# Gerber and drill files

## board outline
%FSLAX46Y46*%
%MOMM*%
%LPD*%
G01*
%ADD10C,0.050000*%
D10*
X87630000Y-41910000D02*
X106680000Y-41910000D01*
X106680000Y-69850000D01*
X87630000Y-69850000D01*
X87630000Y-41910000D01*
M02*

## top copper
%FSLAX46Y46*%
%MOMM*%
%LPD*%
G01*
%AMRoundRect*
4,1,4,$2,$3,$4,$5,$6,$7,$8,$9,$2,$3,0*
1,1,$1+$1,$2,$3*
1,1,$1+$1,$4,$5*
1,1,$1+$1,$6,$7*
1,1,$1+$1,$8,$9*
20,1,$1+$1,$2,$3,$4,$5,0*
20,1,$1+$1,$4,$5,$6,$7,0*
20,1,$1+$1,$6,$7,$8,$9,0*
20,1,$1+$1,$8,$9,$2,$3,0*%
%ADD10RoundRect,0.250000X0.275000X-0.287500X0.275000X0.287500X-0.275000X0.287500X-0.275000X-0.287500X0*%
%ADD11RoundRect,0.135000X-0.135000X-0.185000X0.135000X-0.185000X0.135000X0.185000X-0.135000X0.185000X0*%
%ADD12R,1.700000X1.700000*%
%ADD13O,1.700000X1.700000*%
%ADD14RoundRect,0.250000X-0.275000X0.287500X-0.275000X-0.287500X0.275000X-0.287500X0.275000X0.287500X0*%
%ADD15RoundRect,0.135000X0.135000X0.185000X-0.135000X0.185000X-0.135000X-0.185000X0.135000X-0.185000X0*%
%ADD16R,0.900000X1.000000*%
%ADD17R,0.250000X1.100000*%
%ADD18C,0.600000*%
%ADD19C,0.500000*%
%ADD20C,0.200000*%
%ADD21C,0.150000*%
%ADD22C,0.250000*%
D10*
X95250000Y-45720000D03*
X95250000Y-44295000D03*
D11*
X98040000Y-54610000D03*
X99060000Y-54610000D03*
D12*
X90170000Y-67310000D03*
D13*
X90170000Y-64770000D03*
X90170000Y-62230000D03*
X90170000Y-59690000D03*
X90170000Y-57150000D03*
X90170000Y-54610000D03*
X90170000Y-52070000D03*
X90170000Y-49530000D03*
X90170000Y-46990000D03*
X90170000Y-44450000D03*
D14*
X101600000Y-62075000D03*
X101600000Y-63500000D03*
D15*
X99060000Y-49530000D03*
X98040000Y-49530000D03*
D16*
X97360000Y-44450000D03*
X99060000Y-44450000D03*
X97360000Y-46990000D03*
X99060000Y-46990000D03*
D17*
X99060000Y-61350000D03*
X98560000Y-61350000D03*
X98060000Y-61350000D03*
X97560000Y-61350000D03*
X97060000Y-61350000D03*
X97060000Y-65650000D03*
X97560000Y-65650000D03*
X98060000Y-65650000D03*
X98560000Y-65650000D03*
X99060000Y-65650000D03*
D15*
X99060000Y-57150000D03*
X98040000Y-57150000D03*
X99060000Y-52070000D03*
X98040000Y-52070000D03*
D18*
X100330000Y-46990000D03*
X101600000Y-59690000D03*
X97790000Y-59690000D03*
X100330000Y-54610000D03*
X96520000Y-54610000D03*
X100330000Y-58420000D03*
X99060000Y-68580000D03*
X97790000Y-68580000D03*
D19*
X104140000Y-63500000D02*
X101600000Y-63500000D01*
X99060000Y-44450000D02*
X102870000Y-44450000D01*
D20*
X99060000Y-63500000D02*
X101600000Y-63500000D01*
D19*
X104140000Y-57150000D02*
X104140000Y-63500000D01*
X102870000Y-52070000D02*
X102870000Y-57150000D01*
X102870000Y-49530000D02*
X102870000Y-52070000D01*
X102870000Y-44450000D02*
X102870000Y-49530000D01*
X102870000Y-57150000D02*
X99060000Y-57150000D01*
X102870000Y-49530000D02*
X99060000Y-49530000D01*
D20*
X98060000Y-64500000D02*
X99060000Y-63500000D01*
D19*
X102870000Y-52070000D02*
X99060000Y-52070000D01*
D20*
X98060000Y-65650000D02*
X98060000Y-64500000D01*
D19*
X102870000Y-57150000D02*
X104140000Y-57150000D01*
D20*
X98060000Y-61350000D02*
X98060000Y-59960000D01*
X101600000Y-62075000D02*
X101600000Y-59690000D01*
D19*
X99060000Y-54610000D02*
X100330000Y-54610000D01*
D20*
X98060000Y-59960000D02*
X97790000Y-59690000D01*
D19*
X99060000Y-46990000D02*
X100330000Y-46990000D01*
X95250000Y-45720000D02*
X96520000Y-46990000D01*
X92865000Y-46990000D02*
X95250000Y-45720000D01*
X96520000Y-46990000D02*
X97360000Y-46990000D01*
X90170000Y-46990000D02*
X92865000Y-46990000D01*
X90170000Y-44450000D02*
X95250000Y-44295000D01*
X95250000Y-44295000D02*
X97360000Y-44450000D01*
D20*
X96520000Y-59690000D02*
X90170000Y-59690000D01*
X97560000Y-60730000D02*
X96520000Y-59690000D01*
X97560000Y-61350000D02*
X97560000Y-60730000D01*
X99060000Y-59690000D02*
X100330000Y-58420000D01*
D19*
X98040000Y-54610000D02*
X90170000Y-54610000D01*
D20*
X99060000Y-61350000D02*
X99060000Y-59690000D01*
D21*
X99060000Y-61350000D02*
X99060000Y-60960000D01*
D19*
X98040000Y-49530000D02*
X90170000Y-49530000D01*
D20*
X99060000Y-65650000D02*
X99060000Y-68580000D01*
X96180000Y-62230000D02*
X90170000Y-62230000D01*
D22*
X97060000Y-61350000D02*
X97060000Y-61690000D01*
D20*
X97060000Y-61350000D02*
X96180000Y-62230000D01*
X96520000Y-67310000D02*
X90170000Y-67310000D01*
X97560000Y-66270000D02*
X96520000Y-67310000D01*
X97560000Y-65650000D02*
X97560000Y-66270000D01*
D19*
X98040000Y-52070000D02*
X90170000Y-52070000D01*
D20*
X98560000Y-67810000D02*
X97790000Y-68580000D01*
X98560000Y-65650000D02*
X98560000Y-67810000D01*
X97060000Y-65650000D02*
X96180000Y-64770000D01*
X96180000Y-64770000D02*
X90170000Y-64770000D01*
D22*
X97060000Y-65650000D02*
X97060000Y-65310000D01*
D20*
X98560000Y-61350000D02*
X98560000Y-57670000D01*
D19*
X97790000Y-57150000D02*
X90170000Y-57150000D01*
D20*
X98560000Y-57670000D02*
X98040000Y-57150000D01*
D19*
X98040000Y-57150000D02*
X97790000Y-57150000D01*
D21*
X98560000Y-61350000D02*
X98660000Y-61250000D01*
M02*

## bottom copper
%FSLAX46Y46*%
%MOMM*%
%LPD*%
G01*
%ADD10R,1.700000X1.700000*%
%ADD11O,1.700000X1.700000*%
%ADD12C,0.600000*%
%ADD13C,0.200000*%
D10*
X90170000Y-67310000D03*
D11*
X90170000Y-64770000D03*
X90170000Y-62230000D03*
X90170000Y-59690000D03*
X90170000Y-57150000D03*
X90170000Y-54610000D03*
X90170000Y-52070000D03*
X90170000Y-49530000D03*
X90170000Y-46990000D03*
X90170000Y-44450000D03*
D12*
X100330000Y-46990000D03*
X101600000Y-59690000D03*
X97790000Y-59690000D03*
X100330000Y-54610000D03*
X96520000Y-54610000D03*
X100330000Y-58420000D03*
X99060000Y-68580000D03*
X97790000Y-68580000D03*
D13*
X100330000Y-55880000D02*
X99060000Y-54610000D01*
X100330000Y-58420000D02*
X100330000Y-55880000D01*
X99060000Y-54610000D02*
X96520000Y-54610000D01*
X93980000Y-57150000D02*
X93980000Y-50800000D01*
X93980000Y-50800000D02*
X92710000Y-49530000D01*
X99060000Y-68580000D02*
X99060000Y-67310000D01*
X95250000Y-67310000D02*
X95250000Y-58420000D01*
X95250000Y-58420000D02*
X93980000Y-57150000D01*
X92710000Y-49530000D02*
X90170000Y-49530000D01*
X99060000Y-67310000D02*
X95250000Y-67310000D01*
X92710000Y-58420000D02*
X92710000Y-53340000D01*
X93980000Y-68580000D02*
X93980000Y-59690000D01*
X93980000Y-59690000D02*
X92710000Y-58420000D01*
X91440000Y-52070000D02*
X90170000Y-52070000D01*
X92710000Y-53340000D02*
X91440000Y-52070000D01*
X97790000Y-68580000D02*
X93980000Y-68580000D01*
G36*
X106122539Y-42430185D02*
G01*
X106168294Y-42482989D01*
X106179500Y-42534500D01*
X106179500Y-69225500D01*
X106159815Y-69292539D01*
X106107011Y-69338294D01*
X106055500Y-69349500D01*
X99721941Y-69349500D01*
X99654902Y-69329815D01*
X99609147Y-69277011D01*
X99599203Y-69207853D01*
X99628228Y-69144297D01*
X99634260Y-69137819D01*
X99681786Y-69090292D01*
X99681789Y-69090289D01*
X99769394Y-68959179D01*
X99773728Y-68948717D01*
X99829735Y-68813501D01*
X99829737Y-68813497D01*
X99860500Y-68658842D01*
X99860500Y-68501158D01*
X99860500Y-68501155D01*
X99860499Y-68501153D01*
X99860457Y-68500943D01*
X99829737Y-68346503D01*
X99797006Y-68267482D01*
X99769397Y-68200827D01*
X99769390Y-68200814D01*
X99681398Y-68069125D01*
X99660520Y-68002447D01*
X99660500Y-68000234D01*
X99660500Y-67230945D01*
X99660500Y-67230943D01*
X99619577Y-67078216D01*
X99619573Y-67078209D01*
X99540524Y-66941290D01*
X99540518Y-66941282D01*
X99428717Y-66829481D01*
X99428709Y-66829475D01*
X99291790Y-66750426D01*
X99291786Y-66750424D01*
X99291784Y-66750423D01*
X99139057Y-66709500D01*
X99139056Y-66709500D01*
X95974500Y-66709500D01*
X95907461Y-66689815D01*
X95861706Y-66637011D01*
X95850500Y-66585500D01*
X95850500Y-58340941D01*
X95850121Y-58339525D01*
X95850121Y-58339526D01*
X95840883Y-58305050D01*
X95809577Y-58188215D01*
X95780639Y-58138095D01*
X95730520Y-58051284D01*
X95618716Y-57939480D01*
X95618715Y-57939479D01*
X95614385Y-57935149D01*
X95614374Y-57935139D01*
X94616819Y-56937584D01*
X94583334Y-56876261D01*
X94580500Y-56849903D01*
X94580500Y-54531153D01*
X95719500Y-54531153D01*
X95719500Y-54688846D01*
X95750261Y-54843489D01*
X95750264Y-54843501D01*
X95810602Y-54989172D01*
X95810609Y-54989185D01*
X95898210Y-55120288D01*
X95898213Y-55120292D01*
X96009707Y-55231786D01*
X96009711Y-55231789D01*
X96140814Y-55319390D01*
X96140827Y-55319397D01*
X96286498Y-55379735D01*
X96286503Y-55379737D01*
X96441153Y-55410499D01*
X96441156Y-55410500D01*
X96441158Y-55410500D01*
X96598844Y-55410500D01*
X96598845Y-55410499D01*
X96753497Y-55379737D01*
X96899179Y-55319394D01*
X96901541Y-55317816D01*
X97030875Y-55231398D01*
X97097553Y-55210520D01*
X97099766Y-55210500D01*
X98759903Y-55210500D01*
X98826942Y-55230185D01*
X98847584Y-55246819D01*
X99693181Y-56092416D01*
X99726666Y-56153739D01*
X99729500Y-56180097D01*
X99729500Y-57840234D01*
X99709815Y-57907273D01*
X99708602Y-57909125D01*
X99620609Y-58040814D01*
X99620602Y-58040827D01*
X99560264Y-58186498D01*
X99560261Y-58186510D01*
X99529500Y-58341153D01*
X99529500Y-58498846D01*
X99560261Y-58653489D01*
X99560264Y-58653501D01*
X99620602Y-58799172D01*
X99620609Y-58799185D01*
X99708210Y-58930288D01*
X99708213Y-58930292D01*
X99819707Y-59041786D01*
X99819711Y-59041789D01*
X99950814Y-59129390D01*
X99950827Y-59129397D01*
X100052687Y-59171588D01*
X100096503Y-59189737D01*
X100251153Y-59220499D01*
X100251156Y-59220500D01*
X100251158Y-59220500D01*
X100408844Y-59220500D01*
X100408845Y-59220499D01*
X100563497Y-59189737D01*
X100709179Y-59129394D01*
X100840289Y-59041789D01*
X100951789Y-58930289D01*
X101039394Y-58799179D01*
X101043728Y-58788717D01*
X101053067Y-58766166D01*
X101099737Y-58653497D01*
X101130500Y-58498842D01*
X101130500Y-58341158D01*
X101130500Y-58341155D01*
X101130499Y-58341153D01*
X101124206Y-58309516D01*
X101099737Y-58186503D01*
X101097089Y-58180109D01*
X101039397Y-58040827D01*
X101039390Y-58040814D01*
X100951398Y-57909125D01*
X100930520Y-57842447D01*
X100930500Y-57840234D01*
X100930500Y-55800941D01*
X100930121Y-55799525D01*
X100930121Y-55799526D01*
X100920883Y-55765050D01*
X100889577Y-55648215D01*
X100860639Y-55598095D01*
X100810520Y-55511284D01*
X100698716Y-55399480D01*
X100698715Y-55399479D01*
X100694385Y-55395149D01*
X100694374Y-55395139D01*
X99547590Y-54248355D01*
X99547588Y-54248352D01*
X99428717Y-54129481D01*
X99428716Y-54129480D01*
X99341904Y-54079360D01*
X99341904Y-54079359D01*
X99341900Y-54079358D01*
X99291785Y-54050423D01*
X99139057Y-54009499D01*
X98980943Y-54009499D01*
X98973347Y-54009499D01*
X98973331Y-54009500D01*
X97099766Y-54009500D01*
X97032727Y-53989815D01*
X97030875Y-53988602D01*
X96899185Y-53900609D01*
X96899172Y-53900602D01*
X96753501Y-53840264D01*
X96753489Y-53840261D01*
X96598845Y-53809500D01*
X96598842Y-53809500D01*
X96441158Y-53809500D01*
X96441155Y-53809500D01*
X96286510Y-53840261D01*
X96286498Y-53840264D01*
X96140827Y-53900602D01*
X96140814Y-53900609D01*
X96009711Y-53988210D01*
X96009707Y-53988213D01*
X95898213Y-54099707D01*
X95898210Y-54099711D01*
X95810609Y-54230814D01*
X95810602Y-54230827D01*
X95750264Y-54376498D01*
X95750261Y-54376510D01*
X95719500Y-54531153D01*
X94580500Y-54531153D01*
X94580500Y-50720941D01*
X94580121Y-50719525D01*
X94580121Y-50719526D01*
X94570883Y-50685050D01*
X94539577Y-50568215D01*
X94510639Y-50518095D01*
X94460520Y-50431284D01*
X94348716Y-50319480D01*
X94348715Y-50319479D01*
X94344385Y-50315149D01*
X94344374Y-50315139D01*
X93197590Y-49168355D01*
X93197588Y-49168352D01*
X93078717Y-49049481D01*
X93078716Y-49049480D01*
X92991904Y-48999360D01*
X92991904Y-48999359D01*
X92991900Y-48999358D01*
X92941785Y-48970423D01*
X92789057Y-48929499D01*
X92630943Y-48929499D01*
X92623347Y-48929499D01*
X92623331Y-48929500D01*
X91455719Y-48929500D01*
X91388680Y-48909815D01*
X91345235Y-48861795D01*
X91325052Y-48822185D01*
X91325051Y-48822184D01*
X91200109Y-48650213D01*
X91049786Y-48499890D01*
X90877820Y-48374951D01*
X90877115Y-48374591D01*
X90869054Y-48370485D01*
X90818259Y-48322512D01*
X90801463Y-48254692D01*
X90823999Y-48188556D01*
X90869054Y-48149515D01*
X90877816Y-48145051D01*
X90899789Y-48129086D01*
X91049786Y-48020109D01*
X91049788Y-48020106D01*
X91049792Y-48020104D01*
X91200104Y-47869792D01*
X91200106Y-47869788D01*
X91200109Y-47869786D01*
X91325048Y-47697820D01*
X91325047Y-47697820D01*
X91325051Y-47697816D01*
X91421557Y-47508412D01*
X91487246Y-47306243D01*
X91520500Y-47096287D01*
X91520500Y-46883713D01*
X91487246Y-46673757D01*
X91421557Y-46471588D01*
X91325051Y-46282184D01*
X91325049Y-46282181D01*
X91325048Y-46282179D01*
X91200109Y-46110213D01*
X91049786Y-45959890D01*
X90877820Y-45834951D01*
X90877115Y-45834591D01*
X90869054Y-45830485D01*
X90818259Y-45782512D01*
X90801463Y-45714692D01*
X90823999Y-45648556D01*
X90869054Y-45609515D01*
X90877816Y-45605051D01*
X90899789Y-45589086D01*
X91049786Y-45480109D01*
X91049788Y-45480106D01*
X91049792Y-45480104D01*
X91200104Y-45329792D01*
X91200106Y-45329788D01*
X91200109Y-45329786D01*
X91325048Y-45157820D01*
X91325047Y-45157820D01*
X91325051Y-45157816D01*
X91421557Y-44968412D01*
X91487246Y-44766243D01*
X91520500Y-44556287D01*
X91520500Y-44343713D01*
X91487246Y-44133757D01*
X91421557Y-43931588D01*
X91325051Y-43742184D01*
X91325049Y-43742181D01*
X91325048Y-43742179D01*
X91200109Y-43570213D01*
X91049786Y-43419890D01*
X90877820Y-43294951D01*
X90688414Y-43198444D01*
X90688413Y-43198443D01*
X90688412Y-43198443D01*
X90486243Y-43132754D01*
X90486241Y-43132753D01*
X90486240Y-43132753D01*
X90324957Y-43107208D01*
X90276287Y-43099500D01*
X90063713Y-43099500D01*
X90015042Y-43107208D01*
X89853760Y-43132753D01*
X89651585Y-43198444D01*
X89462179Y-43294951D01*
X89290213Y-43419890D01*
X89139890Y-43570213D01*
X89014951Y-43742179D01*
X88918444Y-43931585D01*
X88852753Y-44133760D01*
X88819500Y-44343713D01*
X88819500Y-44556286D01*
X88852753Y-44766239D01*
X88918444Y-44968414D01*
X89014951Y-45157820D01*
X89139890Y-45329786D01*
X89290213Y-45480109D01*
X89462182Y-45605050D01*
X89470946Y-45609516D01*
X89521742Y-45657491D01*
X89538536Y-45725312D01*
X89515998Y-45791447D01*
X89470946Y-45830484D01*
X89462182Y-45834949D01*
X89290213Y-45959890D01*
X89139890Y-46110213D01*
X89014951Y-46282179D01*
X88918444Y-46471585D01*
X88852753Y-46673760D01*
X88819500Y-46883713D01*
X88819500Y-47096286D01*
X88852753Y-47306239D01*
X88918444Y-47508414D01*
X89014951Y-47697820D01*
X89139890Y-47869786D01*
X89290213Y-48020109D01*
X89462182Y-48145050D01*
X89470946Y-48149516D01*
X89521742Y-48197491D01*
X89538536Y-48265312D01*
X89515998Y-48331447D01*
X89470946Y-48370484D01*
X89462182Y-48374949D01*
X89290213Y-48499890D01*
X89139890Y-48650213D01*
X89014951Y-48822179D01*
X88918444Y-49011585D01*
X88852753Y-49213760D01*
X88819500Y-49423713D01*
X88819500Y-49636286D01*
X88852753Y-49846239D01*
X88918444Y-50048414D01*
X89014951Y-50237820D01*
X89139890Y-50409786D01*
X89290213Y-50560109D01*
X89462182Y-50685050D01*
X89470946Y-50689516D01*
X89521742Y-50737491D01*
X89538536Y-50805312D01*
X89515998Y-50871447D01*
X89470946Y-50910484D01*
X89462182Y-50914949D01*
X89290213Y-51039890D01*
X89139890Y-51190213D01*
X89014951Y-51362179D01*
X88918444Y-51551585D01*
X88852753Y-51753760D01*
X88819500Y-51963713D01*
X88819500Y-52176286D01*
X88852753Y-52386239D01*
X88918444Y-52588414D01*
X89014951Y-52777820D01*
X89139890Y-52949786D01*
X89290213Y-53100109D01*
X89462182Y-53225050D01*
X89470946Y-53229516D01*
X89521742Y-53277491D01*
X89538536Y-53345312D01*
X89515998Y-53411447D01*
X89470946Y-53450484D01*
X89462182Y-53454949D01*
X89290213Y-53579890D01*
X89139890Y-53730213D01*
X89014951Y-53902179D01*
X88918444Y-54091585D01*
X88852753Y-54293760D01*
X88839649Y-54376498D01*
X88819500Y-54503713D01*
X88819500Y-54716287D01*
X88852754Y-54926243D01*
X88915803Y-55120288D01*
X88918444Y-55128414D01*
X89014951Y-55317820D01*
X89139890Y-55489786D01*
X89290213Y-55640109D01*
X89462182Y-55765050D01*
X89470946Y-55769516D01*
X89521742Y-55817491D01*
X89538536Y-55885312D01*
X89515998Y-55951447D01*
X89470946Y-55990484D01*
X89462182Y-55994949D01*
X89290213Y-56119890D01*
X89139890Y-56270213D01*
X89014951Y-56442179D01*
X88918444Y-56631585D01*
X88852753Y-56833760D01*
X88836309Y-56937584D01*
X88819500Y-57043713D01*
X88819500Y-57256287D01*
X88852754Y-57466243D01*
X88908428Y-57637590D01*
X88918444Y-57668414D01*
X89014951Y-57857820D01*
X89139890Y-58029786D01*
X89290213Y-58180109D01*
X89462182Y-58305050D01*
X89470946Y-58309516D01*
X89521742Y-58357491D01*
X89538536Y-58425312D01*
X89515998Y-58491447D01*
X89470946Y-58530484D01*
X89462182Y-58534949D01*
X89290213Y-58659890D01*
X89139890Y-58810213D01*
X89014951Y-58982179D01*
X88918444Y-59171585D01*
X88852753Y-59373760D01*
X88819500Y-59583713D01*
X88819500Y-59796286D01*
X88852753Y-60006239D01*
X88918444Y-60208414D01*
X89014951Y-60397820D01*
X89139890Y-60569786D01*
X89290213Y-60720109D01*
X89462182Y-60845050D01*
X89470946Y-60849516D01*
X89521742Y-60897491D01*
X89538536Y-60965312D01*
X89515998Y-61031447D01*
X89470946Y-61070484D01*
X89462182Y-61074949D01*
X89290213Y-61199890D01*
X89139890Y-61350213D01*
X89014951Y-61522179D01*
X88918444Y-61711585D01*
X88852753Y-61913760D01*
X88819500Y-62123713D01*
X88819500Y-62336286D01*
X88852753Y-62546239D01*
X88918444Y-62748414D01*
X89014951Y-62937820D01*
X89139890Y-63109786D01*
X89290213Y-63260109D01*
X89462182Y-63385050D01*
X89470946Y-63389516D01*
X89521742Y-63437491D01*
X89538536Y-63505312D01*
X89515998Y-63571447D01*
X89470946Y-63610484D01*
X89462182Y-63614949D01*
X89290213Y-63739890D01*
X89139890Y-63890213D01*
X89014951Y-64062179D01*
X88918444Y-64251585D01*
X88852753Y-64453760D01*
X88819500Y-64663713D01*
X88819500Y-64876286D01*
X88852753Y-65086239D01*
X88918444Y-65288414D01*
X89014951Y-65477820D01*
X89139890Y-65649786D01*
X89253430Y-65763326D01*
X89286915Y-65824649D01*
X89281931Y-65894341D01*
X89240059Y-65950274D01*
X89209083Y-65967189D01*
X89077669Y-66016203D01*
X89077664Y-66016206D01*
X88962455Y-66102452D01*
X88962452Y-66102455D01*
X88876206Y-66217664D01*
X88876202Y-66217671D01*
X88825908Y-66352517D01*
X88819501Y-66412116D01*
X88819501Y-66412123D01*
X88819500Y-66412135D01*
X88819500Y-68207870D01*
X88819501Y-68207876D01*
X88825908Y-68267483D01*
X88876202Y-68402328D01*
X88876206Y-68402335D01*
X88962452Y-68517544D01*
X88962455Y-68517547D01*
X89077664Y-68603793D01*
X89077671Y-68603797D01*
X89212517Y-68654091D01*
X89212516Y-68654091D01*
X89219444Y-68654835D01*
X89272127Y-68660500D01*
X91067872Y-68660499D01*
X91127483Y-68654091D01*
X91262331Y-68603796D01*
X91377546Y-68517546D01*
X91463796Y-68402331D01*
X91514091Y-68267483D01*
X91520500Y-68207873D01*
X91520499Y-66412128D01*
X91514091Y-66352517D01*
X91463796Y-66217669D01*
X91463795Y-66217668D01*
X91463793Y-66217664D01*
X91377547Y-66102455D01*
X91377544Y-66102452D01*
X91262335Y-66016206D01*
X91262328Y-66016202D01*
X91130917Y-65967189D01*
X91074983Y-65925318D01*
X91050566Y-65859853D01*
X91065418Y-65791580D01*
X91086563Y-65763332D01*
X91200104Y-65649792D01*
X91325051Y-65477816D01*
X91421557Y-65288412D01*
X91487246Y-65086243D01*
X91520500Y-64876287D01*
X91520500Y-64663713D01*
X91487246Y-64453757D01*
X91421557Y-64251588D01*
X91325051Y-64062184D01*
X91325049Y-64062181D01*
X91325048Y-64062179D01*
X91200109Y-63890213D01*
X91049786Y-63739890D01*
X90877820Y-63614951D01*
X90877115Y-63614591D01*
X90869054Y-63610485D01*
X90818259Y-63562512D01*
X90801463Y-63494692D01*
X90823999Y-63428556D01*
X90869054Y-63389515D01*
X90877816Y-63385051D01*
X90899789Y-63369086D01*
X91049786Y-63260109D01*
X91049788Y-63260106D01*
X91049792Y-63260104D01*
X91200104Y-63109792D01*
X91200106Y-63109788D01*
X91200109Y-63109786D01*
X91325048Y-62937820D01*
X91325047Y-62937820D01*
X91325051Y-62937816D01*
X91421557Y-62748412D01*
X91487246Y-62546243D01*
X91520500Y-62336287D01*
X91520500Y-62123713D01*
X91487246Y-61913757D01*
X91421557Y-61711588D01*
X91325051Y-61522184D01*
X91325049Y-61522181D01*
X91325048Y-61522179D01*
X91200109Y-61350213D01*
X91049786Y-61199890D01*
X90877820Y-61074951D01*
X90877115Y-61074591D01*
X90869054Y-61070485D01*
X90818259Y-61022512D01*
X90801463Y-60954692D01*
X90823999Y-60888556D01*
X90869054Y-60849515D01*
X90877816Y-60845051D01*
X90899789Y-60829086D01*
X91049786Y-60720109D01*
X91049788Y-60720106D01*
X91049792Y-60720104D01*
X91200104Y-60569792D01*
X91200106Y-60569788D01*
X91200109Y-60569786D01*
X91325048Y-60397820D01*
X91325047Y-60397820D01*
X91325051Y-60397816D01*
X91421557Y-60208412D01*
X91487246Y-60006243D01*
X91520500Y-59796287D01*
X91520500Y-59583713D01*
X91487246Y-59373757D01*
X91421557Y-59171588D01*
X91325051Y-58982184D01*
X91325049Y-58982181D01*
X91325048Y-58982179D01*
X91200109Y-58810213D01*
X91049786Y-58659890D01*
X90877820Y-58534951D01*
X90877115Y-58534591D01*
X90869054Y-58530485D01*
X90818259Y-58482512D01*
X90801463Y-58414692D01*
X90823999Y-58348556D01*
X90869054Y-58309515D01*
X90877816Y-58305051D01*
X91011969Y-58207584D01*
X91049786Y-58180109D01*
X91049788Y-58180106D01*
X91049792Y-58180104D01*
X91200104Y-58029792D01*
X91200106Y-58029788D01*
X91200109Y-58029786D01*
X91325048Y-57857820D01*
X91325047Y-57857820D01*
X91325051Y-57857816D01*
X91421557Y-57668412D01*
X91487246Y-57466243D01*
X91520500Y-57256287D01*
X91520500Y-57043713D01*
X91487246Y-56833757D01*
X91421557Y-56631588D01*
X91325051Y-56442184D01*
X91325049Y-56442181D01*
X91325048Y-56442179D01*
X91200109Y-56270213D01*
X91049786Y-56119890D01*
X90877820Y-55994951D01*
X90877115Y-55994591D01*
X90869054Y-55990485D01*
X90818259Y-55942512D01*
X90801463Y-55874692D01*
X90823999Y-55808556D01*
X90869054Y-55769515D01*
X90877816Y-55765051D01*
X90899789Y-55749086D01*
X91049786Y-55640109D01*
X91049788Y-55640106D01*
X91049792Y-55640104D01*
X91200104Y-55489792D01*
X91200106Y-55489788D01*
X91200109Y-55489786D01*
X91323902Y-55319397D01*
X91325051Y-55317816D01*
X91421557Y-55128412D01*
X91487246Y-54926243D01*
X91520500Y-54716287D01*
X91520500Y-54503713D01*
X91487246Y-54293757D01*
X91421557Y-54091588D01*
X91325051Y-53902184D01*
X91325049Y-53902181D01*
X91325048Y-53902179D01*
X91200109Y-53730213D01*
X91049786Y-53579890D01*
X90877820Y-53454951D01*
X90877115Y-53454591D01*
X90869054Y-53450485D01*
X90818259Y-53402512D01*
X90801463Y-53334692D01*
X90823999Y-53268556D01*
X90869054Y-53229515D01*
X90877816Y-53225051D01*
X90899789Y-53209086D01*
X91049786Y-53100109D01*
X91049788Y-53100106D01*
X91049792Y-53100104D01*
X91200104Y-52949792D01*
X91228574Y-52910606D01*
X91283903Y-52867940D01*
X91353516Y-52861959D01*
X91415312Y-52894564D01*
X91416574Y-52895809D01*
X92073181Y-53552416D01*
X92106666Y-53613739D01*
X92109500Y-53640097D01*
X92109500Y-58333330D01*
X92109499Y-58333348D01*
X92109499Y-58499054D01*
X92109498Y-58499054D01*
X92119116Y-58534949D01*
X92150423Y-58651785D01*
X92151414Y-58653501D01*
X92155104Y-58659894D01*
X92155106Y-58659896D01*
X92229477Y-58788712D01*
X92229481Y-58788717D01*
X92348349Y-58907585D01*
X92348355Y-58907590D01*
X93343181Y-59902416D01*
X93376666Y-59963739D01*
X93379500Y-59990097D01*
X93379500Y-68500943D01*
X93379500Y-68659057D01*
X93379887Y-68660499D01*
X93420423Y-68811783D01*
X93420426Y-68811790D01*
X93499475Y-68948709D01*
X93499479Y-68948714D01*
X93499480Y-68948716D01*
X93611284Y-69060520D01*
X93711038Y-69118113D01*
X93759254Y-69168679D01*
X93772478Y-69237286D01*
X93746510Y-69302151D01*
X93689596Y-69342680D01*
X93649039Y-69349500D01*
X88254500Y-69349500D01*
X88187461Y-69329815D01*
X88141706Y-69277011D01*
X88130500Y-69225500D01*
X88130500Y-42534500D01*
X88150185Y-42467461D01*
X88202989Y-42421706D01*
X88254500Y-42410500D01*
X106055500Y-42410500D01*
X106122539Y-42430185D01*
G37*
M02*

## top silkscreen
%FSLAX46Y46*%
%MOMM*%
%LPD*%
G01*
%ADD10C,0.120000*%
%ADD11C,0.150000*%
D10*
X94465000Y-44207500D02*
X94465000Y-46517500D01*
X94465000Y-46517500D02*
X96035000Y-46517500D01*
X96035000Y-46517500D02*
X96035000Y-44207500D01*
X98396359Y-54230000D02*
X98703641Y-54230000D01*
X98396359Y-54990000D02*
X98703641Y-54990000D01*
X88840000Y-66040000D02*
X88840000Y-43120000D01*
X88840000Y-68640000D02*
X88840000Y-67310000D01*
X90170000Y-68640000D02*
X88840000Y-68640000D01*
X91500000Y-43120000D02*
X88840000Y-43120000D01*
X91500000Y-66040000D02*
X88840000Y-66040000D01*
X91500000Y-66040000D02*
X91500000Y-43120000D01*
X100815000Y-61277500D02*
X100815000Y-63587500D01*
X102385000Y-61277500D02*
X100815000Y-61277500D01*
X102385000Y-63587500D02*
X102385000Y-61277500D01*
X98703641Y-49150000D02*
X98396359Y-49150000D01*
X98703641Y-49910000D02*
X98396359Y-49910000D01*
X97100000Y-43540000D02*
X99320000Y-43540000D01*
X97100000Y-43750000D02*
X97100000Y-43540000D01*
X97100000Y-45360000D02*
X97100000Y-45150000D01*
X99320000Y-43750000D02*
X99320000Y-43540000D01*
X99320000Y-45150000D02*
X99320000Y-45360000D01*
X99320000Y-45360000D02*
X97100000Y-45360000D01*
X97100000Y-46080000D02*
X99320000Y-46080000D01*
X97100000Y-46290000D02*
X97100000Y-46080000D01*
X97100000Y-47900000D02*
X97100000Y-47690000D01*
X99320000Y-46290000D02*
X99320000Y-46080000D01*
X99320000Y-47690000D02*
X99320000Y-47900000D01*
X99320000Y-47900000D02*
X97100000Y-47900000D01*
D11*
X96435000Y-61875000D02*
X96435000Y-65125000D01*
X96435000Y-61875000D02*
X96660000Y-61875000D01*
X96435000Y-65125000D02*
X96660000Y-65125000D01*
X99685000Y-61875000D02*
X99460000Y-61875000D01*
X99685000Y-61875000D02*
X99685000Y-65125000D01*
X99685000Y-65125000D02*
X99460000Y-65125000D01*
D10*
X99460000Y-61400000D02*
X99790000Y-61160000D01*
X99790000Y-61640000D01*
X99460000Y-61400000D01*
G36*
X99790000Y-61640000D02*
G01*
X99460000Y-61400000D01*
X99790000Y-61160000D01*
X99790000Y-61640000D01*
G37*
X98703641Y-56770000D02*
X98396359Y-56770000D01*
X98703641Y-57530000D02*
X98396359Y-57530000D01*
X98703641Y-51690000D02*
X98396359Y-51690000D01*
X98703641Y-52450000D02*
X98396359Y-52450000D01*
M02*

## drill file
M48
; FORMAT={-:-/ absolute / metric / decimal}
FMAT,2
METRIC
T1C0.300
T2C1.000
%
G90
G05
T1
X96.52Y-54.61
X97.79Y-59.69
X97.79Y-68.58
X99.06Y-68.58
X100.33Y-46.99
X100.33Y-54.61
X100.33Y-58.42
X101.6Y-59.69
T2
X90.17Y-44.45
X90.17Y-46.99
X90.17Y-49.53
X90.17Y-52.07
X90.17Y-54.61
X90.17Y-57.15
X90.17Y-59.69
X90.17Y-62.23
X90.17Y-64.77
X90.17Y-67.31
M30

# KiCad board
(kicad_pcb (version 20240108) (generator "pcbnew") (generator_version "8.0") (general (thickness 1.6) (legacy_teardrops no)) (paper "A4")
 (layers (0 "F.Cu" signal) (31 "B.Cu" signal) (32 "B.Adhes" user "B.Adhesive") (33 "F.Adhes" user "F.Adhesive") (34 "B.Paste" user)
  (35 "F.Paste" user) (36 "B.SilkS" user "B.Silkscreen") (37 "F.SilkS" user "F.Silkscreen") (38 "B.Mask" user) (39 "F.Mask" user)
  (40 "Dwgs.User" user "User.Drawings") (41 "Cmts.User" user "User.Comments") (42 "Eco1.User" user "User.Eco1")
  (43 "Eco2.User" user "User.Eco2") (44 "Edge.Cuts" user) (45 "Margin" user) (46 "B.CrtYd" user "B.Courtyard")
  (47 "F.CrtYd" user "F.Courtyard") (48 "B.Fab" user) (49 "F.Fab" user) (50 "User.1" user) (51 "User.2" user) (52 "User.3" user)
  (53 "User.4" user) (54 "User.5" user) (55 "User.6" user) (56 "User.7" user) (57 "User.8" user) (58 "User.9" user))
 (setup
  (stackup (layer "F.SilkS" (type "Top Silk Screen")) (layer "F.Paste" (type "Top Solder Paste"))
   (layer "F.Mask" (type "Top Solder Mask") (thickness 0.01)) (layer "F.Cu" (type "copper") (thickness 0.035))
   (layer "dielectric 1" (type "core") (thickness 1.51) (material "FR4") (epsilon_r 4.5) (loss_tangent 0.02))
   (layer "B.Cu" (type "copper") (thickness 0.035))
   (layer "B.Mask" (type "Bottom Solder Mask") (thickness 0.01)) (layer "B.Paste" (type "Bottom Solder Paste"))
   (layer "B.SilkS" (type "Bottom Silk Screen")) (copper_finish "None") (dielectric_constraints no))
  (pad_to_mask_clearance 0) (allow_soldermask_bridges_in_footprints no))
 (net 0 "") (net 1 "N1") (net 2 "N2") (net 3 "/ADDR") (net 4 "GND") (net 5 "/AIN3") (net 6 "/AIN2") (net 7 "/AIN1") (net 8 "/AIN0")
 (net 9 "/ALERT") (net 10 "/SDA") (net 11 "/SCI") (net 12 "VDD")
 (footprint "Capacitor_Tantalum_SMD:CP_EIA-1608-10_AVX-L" (layer "F.Cu") (at 95.25 45.0075 90)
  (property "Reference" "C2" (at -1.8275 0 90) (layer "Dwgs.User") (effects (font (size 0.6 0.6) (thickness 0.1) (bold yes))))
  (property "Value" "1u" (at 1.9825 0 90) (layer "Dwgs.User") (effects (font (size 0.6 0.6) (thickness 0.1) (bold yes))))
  (fp_line (start 0.8 -0.785) (end -1.51 -0.785) (stroke (width 0.12) (type solid)) (layer "F.SilkS"))
  (fp_line (start -1.51 -0.785) (end -1.51 0.785) (stroke (width 0.12) (type solid)) (layer "F.SilkS"))
  (fp_line (start -1.51 0.785) (end 0.8 0.785) (stroke (width 0.12) (type solid)) (layer "F.SilkS"))
  (pad "1" smd roundrect (at -0.7125 0 90) (size 1.075 1.05) (layers "F.Cu" "F.Paste" "F.Mask") (roundrect_rratio 0.238095) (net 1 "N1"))
  (pad "2" smd roundrect (at 0.7125 0 90) (size 1.075 1.05) (layers "F.Cu" "F.Paste" "F.Mask") (roundrect_rratio 0.238095) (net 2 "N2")))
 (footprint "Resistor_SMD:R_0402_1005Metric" (layer "F.Cu") (at 98.55 54.61)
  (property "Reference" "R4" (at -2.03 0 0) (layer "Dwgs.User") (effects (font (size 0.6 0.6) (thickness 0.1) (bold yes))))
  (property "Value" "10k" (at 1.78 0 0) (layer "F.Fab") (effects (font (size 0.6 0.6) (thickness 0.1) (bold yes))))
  (fp_line (start -0.153641 -0.38) (end 0.153641 -0.38) (stroke (width 0.12) (type solid)) (layer "F.SilkS"))
  (fp_line (start -0.153641 0.38) (end 0.153641 0.38) (stroke (width 0.12) (type solid)) (layer "F.SilkS"))
  (pad "1" smd roundrect (at -0.51 0) (size 0.54 0.64) (layers "F.Cu" "F.Paste" "F.Mask") (roundrect_rratio 0.25) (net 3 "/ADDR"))
  (pad "2" smd roundrect (at 0.51 0) (size 0.54 0.64) (layers "F.Cu" "F.Paste" "F.Mask") (roundrect_rratio 0.25) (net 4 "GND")))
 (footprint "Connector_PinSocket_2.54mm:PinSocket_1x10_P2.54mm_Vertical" (layer "F.Cu") (at 90.17 67.31 180)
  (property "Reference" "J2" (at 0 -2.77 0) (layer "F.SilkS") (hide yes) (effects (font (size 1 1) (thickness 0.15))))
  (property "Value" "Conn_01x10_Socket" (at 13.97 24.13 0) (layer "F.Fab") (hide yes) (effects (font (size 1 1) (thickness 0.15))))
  (fp_line (start 1.33 1.27) (end 1.33 24.19) (stroke (width 0.12) (type solid)) (layer "F.SilkS"))
  (fp_line (start 1.33 -1.33) (end 1.33 0) (stroke (width 0.12) (type solid)) (layer "F.SilkS"))
  (fp_line (start 0 -1.33) (end 1.33 -1.33) (stroke (width 0.12) (type solid)) (layer "F.SilkS"))
  (fp_line (start -1.33 24.19) (end 1.33 24.19) (stroke (width 0.12) (type solid)) (layer "F.SilkS"))
  (fp_line (start -1.33 1.27) (end 1.33 1.27) (stroke (width 0.12) (type solid)) (layer "F.SilkS"))
  (fp_line (start -1.33 1.27) (end -1.33 24.19) (stroke (width 0.12) (type solid)) (layer "F.SilkS"))
  (pad "1" thru_hole rect (at 0 0 180) (size 1.7 1.7) (drill 1) (layers "*.Cu" "*.Mask") (remove_unused_layers no) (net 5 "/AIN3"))
  (pad "2" thru_hole oval (at 0 2.54 180) (size 1.7 1.7) (drill 1) (layers "*.Cu" "*.Mask") (remove_unused_layers no) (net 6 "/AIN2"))
  (pad "3" thru_hole oval (at 0 5.08 180) (size 1.7 1.7) (drill 1) (layers "*.Cu" "*.Mask") (remove_unused_layers no) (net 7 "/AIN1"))
  (pad "4" thru_hole oval (at 0 7.62 180) (size 1.7 1.7) (drill 1) (layers "*.Cu" "*.Mask") (remove_unused_layers no) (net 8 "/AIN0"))
  (pad "5" thru_hole oval (at 0 10.16 180) (size 1.7 1.7) (drill 1) (layers "*.Cu" "*.Mask") (remove_unused_layers no) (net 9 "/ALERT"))
  (pad "6" thru_hole oval (at 0 12.7 180) (size 1.7 1.7) (drill 1) (layers "*.Cu" "*.Mask") (remove_unused_layers no) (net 3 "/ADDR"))
  (pad "7" thru_hole oval (at 0 15.24 180) (size 1.7 1.7) (drill 1) (layers "*.Cu" "*.Mask") (remove_unused_layers no) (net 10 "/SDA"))
  (pad "8" thru_hole oval (at 0 17.78 180) (size 1.7 1.7) (drill 1) (layers "*.Cu" "*.Mask") (remove_unused_layers no) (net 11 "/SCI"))
  (pad "9" thru_hole oval (at 0 20.32 180) (size 1.7 1.7) (drill 1) (layers "*.Cu" "*.Mask") (remove_unused_layers no) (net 1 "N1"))
  (pad "10" thru_hole oval (at 0 22.86 180) (size 1.7 1.7) (drill 1) (layers "*.Cu" "*.Mask") (remove_unused_layers no) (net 2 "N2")))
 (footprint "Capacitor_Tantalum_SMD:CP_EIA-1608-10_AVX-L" (layer "F.Cu") (at 101.6 62.7875 -90)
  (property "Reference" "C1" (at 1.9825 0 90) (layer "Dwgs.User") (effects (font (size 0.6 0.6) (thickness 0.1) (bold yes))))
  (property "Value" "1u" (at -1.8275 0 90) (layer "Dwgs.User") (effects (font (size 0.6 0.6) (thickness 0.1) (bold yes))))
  (fp_line (start -1.51 0.785) (end 0.8 0.785) (stroke (width 0.12) (type solid)) (layer "F.SilkS"))
  (fp_line (start -1.51 -0.785) (end -1.51 0.785) (stroke (width 0.12) (type solid)) (layer "F.SilkS"))
  (fp_line (start 0.8 -0.785) (end -1.51 -0.785) (stroke (width 0.12) (type solid)) (layer "F.SilkS"))
  (pad "1" smd roundrect (at -0.7125 0 270) (size 1.075 1.05) (layers "F.Cu" "F.Paste" "F.Mask") (roundrect_rratio 0.238095) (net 4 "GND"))
  (pad "2" smd roundrect (at 0.7125 0 270) (size 1.075 1.05) (layers "F.Cu" "F.Paste" "F.Mask") (roundrect_rratio 0.238095) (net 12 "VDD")))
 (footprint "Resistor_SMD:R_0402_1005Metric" (layer "F.Cu") (at 98.55 49.53 180)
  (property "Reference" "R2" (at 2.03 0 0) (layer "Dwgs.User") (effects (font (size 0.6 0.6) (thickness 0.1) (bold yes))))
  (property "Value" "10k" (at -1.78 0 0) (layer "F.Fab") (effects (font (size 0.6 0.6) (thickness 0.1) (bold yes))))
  (fp_line (start -0.153641 0.38) (end 0.153641 0.38) (stroke (width 0.12) (type solid)) (layer "F.SilkS"))
  (fp_line (start -0.153641 -0.38) (end 0.153641 -0.38) (stroke (width 0.12) (type solid)) (layer "F.SilkS"))
  (pad "1" smd roundrect (at -0.51 0 180) (size 0.54 0.64) (layers "F.Cu" "F.Paste" "F.Mask") (roundrect_rratio 0.25) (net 12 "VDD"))
  (pad "2" smd roundrect (at 0.51 0 180) (size 0.54 0.64) (layers "F.Cu" "F.Paste" "F.Mask") (roundrect_rratio 0.25) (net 11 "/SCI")))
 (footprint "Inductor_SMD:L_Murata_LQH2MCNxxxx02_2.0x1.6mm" (layer "F.Cu") (at 98.21 44.45)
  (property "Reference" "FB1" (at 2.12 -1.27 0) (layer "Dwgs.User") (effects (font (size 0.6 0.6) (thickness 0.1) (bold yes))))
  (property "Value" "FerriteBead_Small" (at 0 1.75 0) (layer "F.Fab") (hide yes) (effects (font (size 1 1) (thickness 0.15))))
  (fp_line (start -1.11 -0.91) (end 1.11 -0.91) (stroke (width 0.12) (type solid)) (layer "F.SilkS"))
  (fp_line (start -1.11 -0.7) (end -1.11 -0.91) (stroke (width 0.12) (type solid)) (layer "F.SilkS"))
  (fp_line (start -1.11 0.91) (end -1.11 0.7) (stroke (width 0.12) (type solid)) (layer "F.SilkS"))
  (fp_line (start 1.11 -0.7) (end 1.11 -0.91) (stroke (width 0.12) (type solid)) (layer "F.SilkS"))
  (fp_line (start 1.11 0.7) (end 1.11 0.91) (stroke (width 0.12) (type solid)) (layer "F.SilkS"))
  (fp_line (start 1.11 0.91) (end -1.11 0.91) (stroke (width 0.12) (type solid)) (layer "F.SilkS"))
  (pad "1" smd rect (at -0.85 0) (size 0.9 1) (layers "F.Cu" "F.Paste" "F.Mask") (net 2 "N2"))
  (pad "2" smd rect (at 0.85 0) (size 0.9 1) (layers "F.Cu" "F.Paste" "F.Mask") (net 12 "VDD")))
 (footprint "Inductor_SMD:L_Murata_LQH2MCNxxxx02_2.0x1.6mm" (layer "F.Cu") (at 98.21 46.99)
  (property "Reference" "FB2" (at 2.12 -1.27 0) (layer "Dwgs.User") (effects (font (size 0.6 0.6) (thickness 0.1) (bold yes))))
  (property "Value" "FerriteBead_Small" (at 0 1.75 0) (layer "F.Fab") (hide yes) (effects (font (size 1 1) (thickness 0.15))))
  (fp_line (start -1.11 -0.91) (end 1.11 -0.91) (stroke (width 0.12) (type solid)) (layer "F.SilkS"))
  (fp_line (start -1.11 -0.7) (end -1.11 -0.91) (stroke (width 0.12) (type solid)) (layer "F.SilkS"))
  (fp_line (start -1.11 0.91) (end -1.11 0.7) (stroke (width 0.12) (type solid)) (layer "F.SilkS"))
  (fp_line (start 1.11 -0.7) (end 1.11 -0.91) (stroke (width 0.12) (type solid)) (layer "F.SilkS"))
  (fp_line (start 1.11 0.7) (end 1.11 0.91) (stroke (width 0.12) (type solid)) (layer "F.SilkS"))
  (fp_line (start 1.11 0.91) (end -1.11 0.91) (stroke (width 0.12) (type solid)) (layer "F.SilkS"))
  (pad "1" smd rect (at -0.85 0) (size 0.9 1) (layers "F.Cu" "F.Paste" "F.Mask") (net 1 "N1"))
  (pad "2" smd rect (at 0.85 0) (size 0.9 1) (layers "F.Cu" "F.Paste" "F.Mask") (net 4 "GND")))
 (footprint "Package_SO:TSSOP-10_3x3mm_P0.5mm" (layer "F.Cu") (at 98.06 63.5 -90)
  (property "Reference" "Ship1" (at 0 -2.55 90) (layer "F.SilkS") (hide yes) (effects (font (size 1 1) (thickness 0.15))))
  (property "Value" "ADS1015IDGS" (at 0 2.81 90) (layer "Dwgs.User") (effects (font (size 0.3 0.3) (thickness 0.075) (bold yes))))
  (fp_line (start -1.625 1.625) (end 1.625 1.625) (stroke (width 0.15) (type solid)) (layer "F.SilkS"))
  (fp_line (start -1.625 1.625) (end -1.625 1.4) (stroke (width 0.15) (type solid)) (layer "F.SilkS"))
  (fp_line (start 1.625 1.625) (end 1.625 1.4) (stroke (width 0.15) (type solid)) (layer "F.SilkS"))
  (fp_line (start -1.625 -1.625) (end -1.625 -1.4) (stroke (width 0.15) (type solid)) (layer "F.SilkS"))
  (fp_line (start -1.625 -1.625) (end 1.625 -1.625) (stroke (width 0.15) (type solid)) (layer "F.SilkS"))
  (fp_line (start 1.625 -1.625) (end 1.625 -1.4) (stroke (width 0.15) (type solid)) (layer "F.SilkS"))
  (fp_poly
   (pts (xy -2.1 -1.4) (xy -2.34 -1.73) (xy -1.86 -1.73) (xy -2.1 -1.4)) (stroke (width 0.12) (type solid)) (fill solid) (layer "F.SilkS"))
  (pad "1" smd rect (at -2.15 -1 270) (size 1.1 0.25) (layers "F.Cu" "F.Paste" "F.Mask") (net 3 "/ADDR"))
  (pad "2" smd rect (at -2.15 -0.5 270) (size 1.1 0.25) (layers "F.Cu" "F.Paste" "F.Mask") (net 9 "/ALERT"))
  (pad "3" smd rect (at -2.15 0 270) (size 1.1 0.25) (layers "F.Cu" "F.Paste" "F.Mask") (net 4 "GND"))
  (pad "4" smd rect (at -2.15 0.5 270) (size 1.1 0.25) (layers "F.Cu" "F.Paste" "F.Mask") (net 8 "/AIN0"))
  (pad "5" smd rect (at -2.15 1 270) (size 1.1 0.25) (layers "F.Cu" "F.Paste" "F.Mask") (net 7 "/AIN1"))
  (pad "6" smd rect (at 2.15 1 270) (size 1.1 0.25) (layers "F.Cu" "F.Paste" "F.Mask") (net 6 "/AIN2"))
  (pad "7" smd rect (at 2.15 0.5 270) (size 1.1 0.25) (layers "F.Cu" "F.Paste" "F.Mask") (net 5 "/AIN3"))
  (pad "8" smd rect (at 2.15 0 270) (size 1.1 0.25) (layers "F.Cu" "F.Paste" "F.Mask") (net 12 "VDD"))
  (pad "9" smd rect (at 2.15 -0.5 270) (size 1.1 0.25) (layers "F.Cu" "F.Paste" "F.Mask") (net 10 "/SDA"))
  (pad "10" smd rect (at 2.15 -1 270) (size 1.1 0.25) (layers "F.Cu" "F.Paste" "F.Mask") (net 11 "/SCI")))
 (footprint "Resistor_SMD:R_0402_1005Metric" (layer "F.Cu") (at 98.55 57.15 180)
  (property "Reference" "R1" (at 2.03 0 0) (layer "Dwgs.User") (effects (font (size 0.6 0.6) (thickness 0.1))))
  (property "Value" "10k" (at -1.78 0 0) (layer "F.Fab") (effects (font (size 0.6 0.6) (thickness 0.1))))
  (fp_line (start -0.153641 0.38) (end 0.153641 0.38) (stroke (width 0.12) (type solid)) (layer "F.SilkS"))
  (fp_line (start -0.153641 -0.38) (end 0.153641 -0.38) (stroke (width 0.12) (type solid)) (layer "F.SilkS"))
  (pad "1" smd roundrect (at -0.51 0 180) (size 0.54 0.64) (layers "F.Cu" "F.Paste" "F.Mask") (roundrect_rratio 0.25) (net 12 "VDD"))
  (pad "2" smd roundrect (at 0.51 0 180) (size 0.54 0.64) (layers "F.Cu" "F.Paste" "F.Mask") (roundrect_rratio 0.25) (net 9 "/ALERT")))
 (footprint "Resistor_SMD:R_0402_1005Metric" (layer "F.Cu") (at 98.55 52.07 180)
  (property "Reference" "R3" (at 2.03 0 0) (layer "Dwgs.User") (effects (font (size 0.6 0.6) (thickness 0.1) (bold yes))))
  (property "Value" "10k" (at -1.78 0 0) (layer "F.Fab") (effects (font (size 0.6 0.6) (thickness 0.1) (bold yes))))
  (fp_line (start -0.153641 0.38) (end 0.153641 0.38) (stroke (width 0.12) (type solid)) (layer "F.SilkS"))
  (fp_line (start -0.153641 -0.38) (end 0.153641 -0.38) (stroke (width 0.12) (type solid)) (layer "F.SilkS"))
  (pad "1" smd roundrect (at -0.51 0 180) (size 0.54 0.64) (layers "F.Cu" "F.Paste" "F.Mask") (roundrect_rratio 0.25) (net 12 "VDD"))
  (pad "2" smd roundrect (at 0.51 0 180) (size 0.54 0.64) (layers "F.Cu" "F.Paste" "F.Mask") (roundrect_rratio 0.25) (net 10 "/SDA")))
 (gr_rect (start 87.63 41.91) (end 106.68 69.85) (stroke (width 0.05) (type default)) (fill none) (layer "Edge.Cuts"))
 (segment (start 104.14 63.5) (end 101.6 63.5) (width 0.5) (layer "F.Cu") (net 12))
 (segment (start 99.06 44.45) (end 102.87 44.45) (width 0.5) (layer "F.Cu") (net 12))
 (segment (start 99.06 63.5) (end 101.6 63.5) (width 0.2) (layer "F.Cu") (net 12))
 (segment (start 104.14 57.15) (end 104.14 63.5) (width 0.5) (layer "F.Cu") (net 12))
 (segment (start 102.87 52.07) (end 102.87 57.15) (width 0.5) (layer "F.Cu") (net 12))
 (segment (start 102.87 49.53) (end 102.87 52.07) (width 0.5) (layer "F.Cu") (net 12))
 (segment (start 102.87 44.45) (end 102.87 49.53) (width 0.5) (layer "F.Cu") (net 12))
 (segment (start 102.87 57.15) (end 99.06 57.15) (width 0.5) (layer "F.Cu") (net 12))
 (segment (start 102.87 49.53) (end 99.06 49.53) (width 0.5) (layer "F.Cu") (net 12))
 (segment (start 98.06 64.5) (end 99.06 63.5) (width 0.2) (layer "F.Cu") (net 12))
 (segment (start 102.87 52.07) (end 99.06 52.07) (width 0.5) (layer "F.Cu") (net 12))
 (segment (start 98.06 65.65) (end 98.06 64.5) (width 0.2) (layer "F.Cu") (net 12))
 (segment (start 102.87 57.15) (end 104.14 57.15) (width 0.5) (layer "F.Cu") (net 12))
 (segment (start 98.06 61.35) (end 98.06 59.96) (width 0.2) (layer "F.Cu") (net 4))
 (segment (start 101.6 62.075) (end 101.6 59.69) (width 0.2) (layer "F.Cu") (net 4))
 (segment (start 99.06 54.61) (end 100.33 54.61) (width 0.5) (layer "F.Cu") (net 4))
 (segment (start 98.06 59.96) (end 97.79 59.69) (width 0.2) (layer "F.Cu") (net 4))
 (segment (start 99.06 46.99) (end 100.33 46.99) (width 0.5) (layer "F.Cu") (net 4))
 (via (at 100.33 46.99) (size 0.6) (drill 0.3) (layers "F.Cu" "B.Cu") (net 4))
 (via (at 101.6 59.69) (size 0.6) (drill 0.3) (layers "F.Cu" "B.Cu") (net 4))
 (via (at 97.79 59.69) (size 0.6) (drill 0.3) (layers "F.Cu" "B.Cu") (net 4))
 (via (at 100.33 54.61) (size 0.6) (drill 0.3) (layers "F.Cu" "B.Cu") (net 4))
 (segment (start 95.25 45.72) (end 96.52 46.99) (width 0.5) (layer "F.Cu") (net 1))
 (segment (start 92.865 46.99) (end 95.25 45.72) (width 0.5) (layer "F.Cu") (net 1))
 (segment (start 96.52 46.99) (end 97.36 46.99) (width 0.5) (layer "F.Cu") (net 1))
 (segment (start 90.17 46.99) (end 92.865 46.99) (width 0.5) (layer "F.Cu") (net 1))
 (segment (start 90.17 44.45) (end 95.25 44.295) (width 0.5) (layer "F.Cu") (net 2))
 (segment (start 95.25 44.295) (end 97.36 44.45) (width 0.5) (layer "F.Cu") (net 2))
 (segment (start 96.52 59.69) (end 90.17 59.69) (width 0.2) (layer "F.Cu") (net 8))
 (segment (start 97.56 60.73) (end 96.52 59.69) (width 0.2) (layer "F.Cu") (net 8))
 (segment (start 97.56 61.35) (end 97.56 60.73) (width 0.2) (layer "F.Cu") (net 8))
 (segment (start 99.06 59.69) (end 100.33 58.42) (width 0.2) (layer "F.Cu") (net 3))
 (segment (start 98.04 54.61) (end 90.17 54.61) (width 0.5) (layer "F.Cu") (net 3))
 (segment (start 99.06 61.35) (end 99.06 59.69) (width 0.2) (layer "F.Cu") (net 3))
 (segment (start 99.06 61.35) (end 99.06 60.96) (width 0.15) (layer "F.Cu") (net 3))
 (via (at 96.52 54.61) (size 0.6) (drill 0.3) (layers "F.Cu" "B.Cu") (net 3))
 (via (at 100.33 58.42) (size 0.6) (drill 0.3) (layers "F.Cu" "B.Cu") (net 3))
 (segment (start 100.33 55.88) (end 99.06 54.61) (width 0.2) (layer "B.Cu") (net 3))
 (segment (start 100.33 58.42) (end 100.33 55.88) (width 0.2) (layer "B.Cu") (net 3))
 (segment (start 99.06 54.61) (end 96.52 54.61) (width 0.2) (layer "B.Cu") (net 3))
 (segment (start 98.04 49.53) (end 90.17 49.53) (width 0.5) (layer "F.Cu") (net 11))
 (segment (start 99.06 65.65) (end 99.06 68.58) (width 0.2) (layer "F.Cu") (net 11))
 (via (at 99.06 68.58) (size 0.6) (drill 0.3) (layers "F.Cu" "B.Cu") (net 11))
 (segment (start 93.98 57.15) (end 93.98 50.8) (width 0.2) (layer "B.Cu") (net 11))
 (segment (start 93.98 50.8) (end 92.71 49.53) (width 0.2) (layer "B.Cu") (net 11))
 (segment (start 99.06 68.58) (end 99.06 67.31) (width 0.2) (layer "B.Cu") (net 11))
 (segment (start 95.25 67.31) (end 95.25 58.42) (width 0.2) (layer "B.Cu") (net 11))
 (segment (start 95.25 58.42) (end 93.98 57.15) (width 0.2) (layer "B.Cu") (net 11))
 (segment (start 92.71 49.53) (end 90.17 49.53) (width 0.2) (layer "B.Cu") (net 11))
 (segment (start 99.06 67.31) (end 95.25 67.31) (width 0.2) (layer "B.Cu") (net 11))
 (segment (start 96.18 62.23) (end 90.17 62.23) (width 0.2) (layer "F.Cu") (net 7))
 (segment (start 97.06 61.35) (end 97.06 61.69) (width 0.25) (layer "F.Cu") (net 7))
 (segment (start 97.06 61.35) (end 96.18 62.23) (width 0.2) (layer "F.Cu") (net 7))
 (segment (start 96.52 67.31) (end 90.17 67.31) (width 0.2) (layer "F.Cu") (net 5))
 (segment (start 97.56 66.27) (end 96.52 67.31) (width 0.2) (layer "F.Cu") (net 5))
 (segment (start 97.56 65.65) (end 97.56 66.27) (width 0.2) (layer "F.Cu") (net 5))
 (segment (start 98.04 52.07) (end 90.17 52.07) (width 0.5) (layer "F.Cu") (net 10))
 (segment (start 98.56 67.81) (end 97.79 68.58) (width 0.2) (layer "F.Cu") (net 10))
 (segment (start 98.56 65.65) (end 98.56 67.81) (width 0.2) (layer "F.Cu") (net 10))
 (via (at 97.79 68.58) (size 0.6) (drill 0.3) (layers "F.Cu" "B.Cu") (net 10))
 (segment (start 92.71 58.42) (end 92.71 53.34) (width 0.2) (layer "B.Cu") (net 10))
 (segment (start 93.98 68.58) (end 93.98 59.69) (width 0.2) (layer "B.Cu") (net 10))
 (segment (start 93.98 59.69) (end 92.71 58.42) (width 0.2) (layer "B.Cu") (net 10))
 (segment (start 91.44 52.07) (end 90.17 52.07) (width 0.2) (layer "B.Cu") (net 10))
 (segment (start 92.71 53.34) (end 91.44 52.07) (width 0.2) (layer "B.Cu") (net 10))
 (segment (start 97.79 68.58) (end 93.98 68.58) (width 0.2) (layer "B.Cu") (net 10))
 (segment (start 97.06 65.65) (end 96.18 64.77) (width 0.2) (layer "F.Cu") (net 6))
 (segment (start 96.18 64.77) (end 90.17 64.77) (width 0.2) (layer "F.Cu") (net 6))
 (segment (start 97.06 65.65) (end 97.06 65.31) (width 0.25) (layer "F.Cu") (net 6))
 (segment (start 98.56 61.35) (end 98.56 57.67) (width 0.2) (layer "F.Cu") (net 9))
 (segment (start 97.79 57.15) (end 90.17 57.15) (width 0.5) (layer "F.Cu") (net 9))
 (segment (start 98.56 57.67) (end 98.04 57.15) (width 0.2) (layer "F.Cu") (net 9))
 (segment (start 98.04 57.15) (end 97.79 57.15) (width 0.5) (layer "F.Cu") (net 9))
 (segment (start 98.56 61.35) (end 98.66 61.25) (width 0.15) (layer "F.Cu") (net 9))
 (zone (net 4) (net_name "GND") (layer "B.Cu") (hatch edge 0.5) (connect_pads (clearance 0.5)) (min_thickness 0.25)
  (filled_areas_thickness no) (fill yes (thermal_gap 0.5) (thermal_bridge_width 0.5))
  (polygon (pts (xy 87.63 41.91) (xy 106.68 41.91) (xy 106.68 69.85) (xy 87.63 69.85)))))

